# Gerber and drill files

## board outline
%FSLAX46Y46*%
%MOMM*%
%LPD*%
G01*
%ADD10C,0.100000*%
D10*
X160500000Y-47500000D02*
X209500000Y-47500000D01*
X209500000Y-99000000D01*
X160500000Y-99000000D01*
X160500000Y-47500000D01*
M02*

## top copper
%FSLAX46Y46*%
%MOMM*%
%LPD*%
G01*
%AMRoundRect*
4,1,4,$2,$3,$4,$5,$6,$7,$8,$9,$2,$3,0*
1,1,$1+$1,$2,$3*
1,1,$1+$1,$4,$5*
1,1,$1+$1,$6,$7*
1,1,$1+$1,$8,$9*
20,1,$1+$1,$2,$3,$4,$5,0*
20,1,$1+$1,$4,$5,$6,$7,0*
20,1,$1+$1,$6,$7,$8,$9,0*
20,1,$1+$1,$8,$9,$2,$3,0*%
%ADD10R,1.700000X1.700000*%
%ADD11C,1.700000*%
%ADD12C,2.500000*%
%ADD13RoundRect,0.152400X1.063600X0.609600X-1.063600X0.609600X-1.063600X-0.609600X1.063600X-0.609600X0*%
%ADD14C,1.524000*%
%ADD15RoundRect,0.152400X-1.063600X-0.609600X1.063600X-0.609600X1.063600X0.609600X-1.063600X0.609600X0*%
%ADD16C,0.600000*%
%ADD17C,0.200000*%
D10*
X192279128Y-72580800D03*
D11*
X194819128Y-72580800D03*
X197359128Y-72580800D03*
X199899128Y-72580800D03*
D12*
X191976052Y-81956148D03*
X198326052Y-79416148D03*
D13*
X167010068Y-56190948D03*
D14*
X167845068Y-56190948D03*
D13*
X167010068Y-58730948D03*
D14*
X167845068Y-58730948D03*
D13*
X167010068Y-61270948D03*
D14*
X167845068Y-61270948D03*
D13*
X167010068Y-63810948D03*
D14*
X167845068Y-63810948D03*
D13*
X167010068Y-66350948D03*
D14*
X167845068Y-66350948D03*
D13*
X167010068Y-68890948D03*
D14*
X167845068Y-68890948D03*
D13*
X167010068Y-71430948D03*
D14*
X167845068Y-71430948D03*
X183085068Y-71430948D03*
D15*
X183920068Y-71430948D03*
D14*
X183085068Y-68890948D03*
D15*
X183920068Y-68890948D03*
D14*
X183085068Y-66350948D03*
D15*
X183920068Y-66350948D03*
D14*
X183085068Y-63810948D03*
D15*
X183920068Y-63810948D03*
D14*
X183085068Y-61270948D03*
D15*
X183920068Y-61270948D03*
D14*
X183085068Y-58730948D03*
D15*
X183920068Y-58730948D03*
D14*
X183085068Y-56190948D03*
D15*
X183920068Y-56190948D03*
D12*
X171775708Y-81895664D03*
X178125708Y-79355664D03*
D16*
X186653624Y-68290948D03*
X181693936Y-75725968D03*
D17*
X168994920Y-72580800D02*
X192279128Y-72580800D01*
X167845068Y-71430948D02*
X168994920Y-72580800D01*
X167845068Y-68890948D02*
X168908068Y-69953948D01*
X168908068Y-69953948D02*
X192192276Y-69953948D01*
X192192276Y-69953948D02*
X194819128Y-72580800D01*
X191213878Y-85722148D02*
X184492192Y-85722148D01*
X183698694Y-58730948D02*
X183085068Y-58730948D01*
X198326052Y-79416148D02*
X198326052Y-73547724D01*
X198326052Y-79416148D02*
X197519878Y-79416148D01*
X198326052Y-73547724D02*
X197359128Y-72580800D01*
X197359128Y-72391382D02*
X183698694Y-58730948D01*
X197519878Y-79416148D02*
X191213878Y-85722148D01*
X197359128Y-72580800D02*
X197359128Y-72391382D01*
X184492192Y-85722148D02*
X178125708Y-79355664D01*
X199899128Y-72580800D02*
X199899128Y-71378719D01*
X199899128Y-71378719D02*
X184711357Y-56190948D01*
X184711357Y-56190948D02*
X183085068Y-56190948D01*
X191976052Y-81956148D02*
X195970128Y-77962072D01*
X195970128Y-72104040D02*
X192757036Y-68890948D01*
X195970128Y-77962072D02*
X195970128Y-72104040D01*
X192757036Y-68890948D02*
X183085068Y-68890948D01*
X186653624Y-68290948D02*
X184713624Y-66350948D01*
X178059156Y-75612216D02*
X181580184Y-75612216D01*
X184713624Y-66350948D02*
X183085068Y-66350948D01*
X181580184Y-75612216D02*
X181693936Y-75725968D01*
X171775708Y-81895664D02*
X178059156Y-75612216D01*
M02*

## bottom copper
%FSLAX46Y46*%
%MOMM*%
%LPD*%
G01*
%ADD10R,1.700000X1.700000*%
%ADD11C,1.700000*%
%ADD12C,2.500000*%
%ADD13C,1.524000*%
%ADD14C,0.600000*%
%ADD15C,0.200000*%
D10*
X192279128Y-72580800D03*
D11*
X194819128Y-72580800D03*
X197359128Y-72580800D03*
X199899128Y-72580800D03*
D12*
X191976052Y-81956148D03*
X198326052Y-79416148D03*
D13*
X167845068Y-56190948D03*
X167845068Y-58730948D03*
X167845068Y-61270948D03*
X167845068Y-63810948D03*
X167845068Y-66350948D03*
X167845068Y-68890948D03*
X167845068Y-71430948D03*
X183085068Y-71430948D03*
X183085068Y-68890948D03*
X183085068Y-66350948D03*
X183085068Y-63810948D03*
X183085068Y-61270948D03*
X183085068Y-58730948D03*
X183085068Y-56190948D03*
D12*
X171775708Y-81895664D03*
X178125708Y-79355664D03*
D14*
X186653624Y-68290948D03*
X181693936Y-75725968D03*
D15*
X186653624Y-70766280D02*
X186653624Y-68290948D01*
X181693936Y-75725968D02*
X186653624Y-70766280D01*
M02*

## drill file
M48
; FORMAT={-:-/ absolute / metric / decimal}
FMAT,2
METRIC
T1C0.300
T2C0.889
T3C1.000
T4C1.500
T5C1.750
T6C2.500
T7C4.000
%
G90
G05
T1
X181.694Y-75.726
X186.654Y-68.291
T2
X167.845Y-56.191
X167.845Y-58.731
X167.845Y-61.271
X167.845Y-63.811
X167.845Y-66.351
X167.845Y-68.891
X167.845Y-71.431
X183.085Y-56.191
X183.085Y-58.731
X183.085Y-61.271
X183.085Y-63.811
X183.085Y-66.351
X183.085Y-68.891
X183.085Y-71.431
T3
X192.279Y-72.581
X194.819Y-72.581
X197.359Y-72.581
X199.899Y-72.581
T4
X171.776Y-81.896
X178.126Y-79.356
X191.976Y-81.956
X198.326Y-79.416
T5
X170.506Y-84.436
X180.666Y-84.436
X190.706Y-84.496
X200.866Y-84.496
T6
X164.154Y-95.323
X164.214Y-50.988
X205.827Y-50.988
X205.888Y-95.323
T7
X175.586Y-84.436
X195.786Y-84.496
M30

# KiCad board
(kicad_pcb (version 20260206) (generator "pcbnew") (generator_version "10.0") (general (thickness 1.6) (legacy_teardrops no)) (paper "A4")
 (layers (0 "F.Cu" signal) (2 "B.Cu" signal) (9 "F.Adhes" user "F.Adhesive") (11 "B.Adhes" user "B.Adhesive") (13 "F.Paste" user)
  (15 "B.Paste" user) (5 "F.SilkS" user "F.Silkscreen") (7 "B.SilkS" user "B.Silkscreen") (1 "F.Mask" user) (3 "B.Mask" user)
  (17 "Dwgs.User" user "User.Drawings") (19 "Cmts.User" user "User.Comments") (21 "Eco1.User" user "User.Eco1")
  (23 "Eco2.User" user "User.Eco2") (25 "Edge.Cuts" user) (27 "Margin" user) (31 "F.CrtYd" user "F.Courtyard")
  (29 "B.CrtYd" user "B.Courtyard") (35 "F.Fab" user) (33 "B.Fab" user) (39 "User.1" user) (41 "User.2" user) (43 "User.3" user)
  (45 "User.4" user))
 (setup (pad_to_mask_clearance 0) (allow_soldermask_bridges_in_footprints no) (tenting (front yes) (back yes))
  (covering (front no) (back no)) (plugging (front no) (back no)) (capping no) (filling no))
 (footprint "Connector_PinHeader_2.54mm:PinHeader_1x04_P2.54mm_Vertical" (layer "F.Cu") (at 192.279128 72.5808 90)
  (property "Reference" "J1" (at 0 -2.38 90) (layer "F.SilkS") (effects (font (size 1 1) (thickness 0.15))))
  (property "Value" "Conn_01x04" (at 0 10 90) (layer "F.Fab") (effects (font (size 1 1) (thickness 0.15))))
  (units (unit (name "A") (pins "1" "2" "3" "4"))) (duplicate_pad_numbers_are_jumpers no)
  (pad "1" thru_hole rect (at 0 0 90) (size 1.7 1.7) (drill 1) (layers "*.Cu" "*.Mask") (remove_unused_layers no) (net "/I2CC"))
  (pad "2" thru_hole circle (at 0 2.54 90) (size 1.7 1.7) (drill 1) (layers "*.Cu" "*.Mask") (remove_unused_layers no) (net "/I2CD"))
  (pad "3" thru_hole circle (at 0 5.08 90) (size 1.7 1.7) (drill 1) (layers "*.Cu" "*.Mask") (remove_unused_layers no) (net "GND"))
  (pad "4" thru_hole circle (at 0 7.62 90) (size 1.7 1.7) (drill 1) (layers "*.Cu" "*.Mask") (remove_unused_layers no) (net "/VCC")))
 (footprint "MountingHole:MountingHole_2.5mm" (layer "F.Cu") (at 164.21406 50.988012)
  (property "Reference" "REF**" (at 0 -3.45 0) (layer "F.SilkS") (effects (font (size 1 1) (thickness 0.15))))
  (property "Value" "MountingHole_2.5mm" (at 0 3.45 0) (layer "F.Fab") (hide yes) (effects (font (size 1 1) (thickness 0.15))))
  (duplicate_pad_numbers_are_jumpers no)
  (pad "" np_thru_hole circle (at 0 0) (size 2.5 2.5) (drill 2.5) (layers "*.Cu" "*.Mask")))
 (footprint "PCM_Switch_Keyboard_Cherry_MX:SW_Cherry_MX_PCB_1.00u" (layer "F.Cu") (at 195.786052 84.496148)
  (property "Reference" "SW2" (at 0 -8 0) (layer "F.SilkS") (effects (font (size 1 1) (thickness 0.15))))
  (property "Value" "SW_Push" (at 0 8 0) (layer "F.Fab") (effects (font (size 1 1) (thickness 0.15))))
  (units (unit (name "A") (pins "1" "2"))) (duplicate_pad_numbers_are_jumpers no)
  (pad "" np_thru_hole circle (at -5.08 0) (size 1.75 1.75) (drill 1.75) (layers "*.Cu" "*.Mask"))
  (pad "" np_thru_hole circle (at 0 0) (size 4 4) (drill 4) (layers "*.Cu" "*.Mask"))
  (pad "" np_thru_hole circle (at 5.08 0) (size 1.75 1.75) (drill 1.75) (layers "*.Cu" "*.Mask"))
  (pad "1" thru_hole circle (at -3.81 -2.54) (size 2.5 2.5) (drill 1.5) (layers "*.Cu" "*.Mask") (remove_unused_layers no)
   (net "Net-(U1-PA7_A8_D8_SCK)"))
  (pad "2" thru_hole circle (at 2.54 -5.08) (size 2.5 2.5) (drill 1.5) (layers "*.Cu" "*.Mask") (remove_unused_layers no) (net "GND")))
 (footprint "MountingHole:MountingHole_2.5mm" (layer "F.Cu") (at 164.153576 95.322784)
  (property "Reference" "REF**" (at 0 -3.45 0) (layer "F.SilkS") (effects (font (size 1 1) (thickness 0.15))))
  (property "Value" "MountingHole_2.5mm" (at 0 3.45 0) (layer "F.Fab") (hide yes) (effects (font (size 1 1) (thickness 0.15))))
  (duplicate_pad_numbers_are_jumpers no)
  (pad "" np_thru_hole circle (at 0 0) (size 2.5 2.5) (drill 2.5) (layers "*.Cu" "*.Mask")))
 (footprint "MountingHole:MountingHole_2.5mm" (layer "F.Cu") (at 205.827052 50.988012)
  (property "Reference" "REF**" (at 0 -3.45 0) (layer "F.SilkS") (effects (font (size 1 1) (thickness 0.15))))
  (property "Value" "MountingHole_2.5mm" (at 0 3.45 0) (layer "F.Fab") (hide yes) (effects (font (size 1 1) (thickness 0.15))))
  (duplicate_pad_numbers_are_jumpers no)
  (pad "" np_thru_hole circle (at 0 0) (size 2.5 2.5) (drill 2.5) (layers "*.Cu" "*.Mask")))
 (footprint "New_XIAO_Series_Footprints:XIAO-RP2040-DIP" (layer "F.Cu") (at 175.465068 63.810948 90)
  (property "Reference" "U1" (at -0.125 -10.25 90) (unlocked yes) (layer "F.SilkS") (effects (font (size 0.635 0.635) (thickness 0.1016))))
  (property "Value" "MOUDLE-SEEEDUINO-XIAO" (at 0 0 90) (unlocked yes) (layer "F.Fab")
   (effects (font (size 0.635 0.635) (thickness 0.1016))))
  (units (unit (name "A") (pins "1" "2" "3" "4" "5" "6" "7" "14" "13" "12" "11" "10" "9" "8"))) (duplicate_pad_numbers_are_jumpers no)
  (pad "1" smd roundrect (at 7.62 -8.455 180) (size 2.432 1.524) (layers "F.Cu" "F.Mask") (roundrect_rratio 0.1)
   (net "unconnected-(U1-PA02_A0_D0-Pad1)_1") (thermal_bridge_angle 45))
  (pad "1" thru_hole circle (at 7.62 -7.62 180) (size 1.524 1.524) (drill 0.889) (layers "*.Cu" "*.Mask") (remove_unused_layers no)
   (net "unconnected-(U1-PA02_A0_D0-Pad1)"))
  (pad "2" smd roundrect (at 5.08 -8.455 180) (size 2.432 1.524) (layers "F.Cu" "F.Mask") (roundrect_rratio 0.1)
   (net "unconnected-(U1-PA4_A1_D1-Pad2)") (thermal_bridge_angle 45))
  (pad "2" thru_hole circle (at 5.08 -7.62 180) (size 1.524 1.524) (drill 0.889) (layers "*.Cu" "*.Mask") (remove_unused_layers no)
   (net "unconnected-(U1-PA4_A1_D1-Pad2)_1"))
  (pad "3" smd roundrect (at 2.54 -8.455 180) (size 2.432 1.524) (layers "F.Cu" "F.Mask") (roundrect_rratio 0.1)
   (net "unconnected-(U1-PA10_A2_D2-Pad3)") (thermal_bridge_angle 45))
  (pad "3" thru_hole circle (at 2.54 -7.62 180) (size 1.524 1.524) (drill 0.889) (layers "*.Cu" "*.Mask") (remove_unused_layers no)
   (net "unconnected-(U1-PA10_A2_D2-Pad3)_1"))
  (pad "4" smd roundrect (at 0 -8.455 180) (size 2.432 1.524) (layers "F.Cu" "F.Mask") (roundrect_rratio 0.1)
   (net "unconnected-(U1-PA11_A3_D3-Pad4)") (thermal_bridge_angle 45))
  (pad "4" thru_hole circle (at 0 -7.62 180) (size 1.524 1.524) (drill 0.889) (layers "*.Cu" "*.Mask") (remove_unused_layers no)
   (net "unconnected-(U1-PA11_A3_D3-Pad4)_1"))
  (pad "5" smd roundrect (at -2.54 -8.455 180) (size 2.432 1.524) (layers "F.Cu" "F.Mask") (roundrect_rratio 0.1)
   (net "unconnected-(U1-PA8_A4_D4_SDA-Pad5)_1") (thermal_bridge_angle 45))
  (pad "5" thru_hole circle (at -2.54 -7.62 180) (size 1.524 1.524) (drill 0.889) (layers "*.Cu" "*.Mask") (remove_unused_layers no)
   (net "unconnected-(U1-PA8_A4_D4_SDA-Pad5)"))
  (pad "6" smd roundrect (at -5.08 -8.455 180) (size 2.432 1.524) (layers "F.Cu" "F.Mask") (roundrect_rratio 0.1) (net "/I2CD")
   (thermal_bridge_angle 45))
  (pad "6" thru_hole circle (at -5.08 -7.62 180) (size 1.524 1.524) (drill 0.889) (layers "*.Cu" "*.Mask") (remove_unused_layers no)
   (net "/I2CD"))
  (pad "7" smd roundrect (at -7.62 -8.455 180) (size 2.432 1.524) (layers "F.Cu" "F.Mask") (roundrect_rratio 0.1) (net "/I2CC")
   (thermal_bridge_angle 45))
  (pad "7" thru_hole circle (at -7.62 -7.62 180) (size 1.524 1.524) (drill 0.889) (layers "*.Cu" "*.Mask") (remove_unused_layers no)
   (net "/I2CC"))
  (pad "8" thru_hole circle (at -7.62 7.62) (size 1.524 1.524) (drill 0.889) (layers "*.Cu" "*.Mask") (remove_unused_layers no)
   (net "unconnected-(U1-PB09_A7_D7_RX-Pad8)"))
  (pad "8" smd roundrect (at -7.62 8.455) (size 2.432 1.524) (layers "F.Cu" "F.Mask") (roundrect_rratio 0.1)
   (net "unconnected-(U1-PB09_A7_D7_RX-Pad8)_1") (thermal_bridge_angle 45))
  (pad "9" thru_hole circle (at -5.08 7.62) (size 1.524 1.524) (drill 0.889) (layers "*.Cu" "*.Mask") (remove_unused_layers no)
   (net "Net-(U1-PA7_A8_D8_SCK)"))
  (pad "9" smd roundrect (at -5.08 8.455) (size 2.432 1.524) (layers "F.Cu" "F.Mask") (roundrect_rratio 0.1) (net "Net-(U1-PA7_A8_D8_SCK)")
   (thermal_bridge_angle 45))
  (pad "10" thru_hole circle (at -2.54 7.62) (size 1.524 1.524) (drill 0.889) (layers "*.Cu" "*.Mask") (remove_unused_layers no)
   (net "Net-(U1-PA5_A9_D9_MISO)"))
  (pad "10" smd roundrect (at -2.54 8.455) (size 2.432 1.524) (layers "F.Cu" "F.Mask") (roundrect_rratio 0.1)
   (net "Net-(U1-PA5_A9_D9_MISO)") (thermal_bridge_angle 45))
  (pad "11" thru_hole circle (at 0 7.62) (size 1.524 1.524) (drill 0.889) (layers "*.Cu" "*.Mask") (remove_unused_layers no)
   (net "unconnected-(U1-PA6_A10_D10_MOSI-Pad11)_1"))
  (pad "11" smd roundrect (at 0 8.455) (size 2.432 1.524) (layers "F.Cu" "F.Mask") (roundrect_rratio 0.1)
   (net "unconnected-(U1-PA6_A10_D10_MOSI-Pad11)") (thermal_bridge_angle 45))
  (pad "12" thru_hole circle (at 2.54 7.62) (size 1.524 1.524) (drill 0.889) (layers "*.Cu" "*.Mask") (remove_unused_layers no)
   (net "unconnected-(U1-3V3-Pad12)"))
  (pad "12" smd roundrect (at 2.54 8.455) (size 2.432 1.524) (layers "F.Cu" "F.Mask") (roundrect_rratio 0.1)
   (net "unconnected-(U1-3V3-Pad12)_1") (thermal_bridge_angle 45))
  (pad "13" thru_hole circle (at 5.08 7.62) (size 1.524 1.524) (drill 0.889) (layers "*.Cu" "*.Mask") (remove_unused_layers no) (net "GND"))
  (pad "13" smd roundrect (at 5.08 8.455) (size 2.432 1.524) (layers "F.Cu" "F.Mask") (roundrect_rratio 0.1) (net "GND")
   (thermal_bridge_angle 45))
  (pad "14" thru_hole circle (at 7.62 7.62) (size 1.524 1.524) (drill 0.889) (layers "*.Cu" "*.Mask") (remove_unused_layers no) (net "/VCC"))
  (pad "14" smd roundrect (at 7.62 8.455) (size 2.432 1.524) (layers "F.Cu" "F.Mask") (roundrect_rratio 0.1) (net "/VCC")
   (thermal_bridge_angle 45)))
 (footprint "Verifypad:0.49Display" (layer "F.Cu") (at 193.609284 63.20578)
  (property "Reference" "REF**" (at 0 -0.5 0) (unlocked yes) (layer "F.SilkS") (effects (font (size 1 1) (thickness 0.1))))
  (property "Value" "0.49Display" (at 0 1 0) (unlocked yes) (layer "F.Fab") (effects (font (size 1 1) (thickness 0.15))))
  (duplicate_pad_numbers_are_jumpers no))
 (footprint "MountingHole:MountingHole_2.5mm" (layer "F.Cu") (at 205.887536 95.322784)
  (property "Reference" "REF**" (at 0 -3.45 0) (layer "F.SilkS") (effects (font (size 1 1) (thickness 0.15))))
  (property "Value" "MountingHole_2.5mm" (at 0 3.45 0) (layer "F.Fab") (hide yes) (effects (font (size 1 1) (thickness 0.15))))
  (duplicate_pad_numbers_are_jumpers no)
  (pad "" np_thru_hole circle (at 0 0) (size 2.5 2.5) (drill 2.5) (layers "*.Cu" "*.Mask")))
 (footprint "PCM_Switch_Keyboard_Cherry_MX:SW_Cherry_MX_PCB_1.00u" (layer "F.Cu") (at 175.585708 84.435664)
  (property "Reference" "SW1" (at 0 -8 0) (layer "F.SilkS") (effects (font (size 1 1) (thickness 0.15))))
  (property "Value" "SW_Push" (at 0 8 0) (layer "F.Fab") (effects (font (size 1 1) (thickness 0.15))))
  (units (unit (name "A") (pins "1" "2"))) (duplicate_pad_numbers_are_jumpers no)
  (pad "" np_thru_hole circle (at -5.08 0) (size 1.75 1.75) (drill 1.75) (layers "*.Cu" "*.Mask"))
  (pad "" np_thru_hole circle (at 0 0) (size 4 4) (drill 4) (layers "*.Cu" "*.Mask"))
  (pad "" np_thru_hole circle (at 5.08 0) (size 1.75 1.75) (drill 1.75) (layers "*.Cu" "*.Mask"))
  (pad "1" thru_hole circle (at -3.81 -2.54) (size 2.5 2.5) (drill 1.5) (layers "*.Cu" "*.Mask") (remove_unused_layers no)
   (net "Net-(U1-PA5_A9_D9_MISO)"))
  (pad "2" thru_hole circle (at 2.54 -5.08) (size 2.5 2.5) (drill 1.5) (layers "*.Cu" "*.Mask") (remove_unused_layers no) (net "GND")))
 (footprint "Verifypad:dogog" (layer "B.Cu") (at 175.734887 92.160269 180)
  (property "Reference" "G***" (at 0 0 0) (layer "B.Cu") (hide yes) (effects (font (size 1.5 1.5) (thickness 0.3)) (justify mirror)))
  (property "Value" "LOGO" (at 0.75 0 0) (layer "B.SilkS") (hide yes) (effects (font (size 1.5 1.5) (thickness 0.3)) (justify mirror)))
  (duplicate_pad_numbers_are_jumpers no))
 (gr_rect (start 160.5 47.5) (end 209.5 99) (stroke (width 0.1) (type solid)) (fill no) (layer "Edge.Cuts"))
 (segment (start 168.99492 72.5808) (end 192.279128 72.5808) (width 0.2) (layer "F.Cu") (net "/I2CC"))
 (segment (start 167.845068 71.430948) (end 168.99492 72.5808) (width 0.2) (layer "F.Cu") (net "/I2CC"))
 (segment (start 167.845068 68.890948) (end 168.908068 69.953948) (width 0.2) (layer "F.Cu") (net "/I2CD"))
 (segment (start 168.908068 69.953948) (end 192.192276 69.953948) (width 0.2) (layer "F.Cu") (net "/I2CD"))
 (segment (start 192.192276 69.953948) (end 194.819128 72.5808) (width 0.2) (layer "F.Cu") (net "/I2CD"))
 (segment (start 191.213878 85.722148) (end 184.492192 85.722148) (width 0.2) (layer "F.Cu") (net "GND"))
 (segment (start 183.698694 58.730948) (end 183.085068 58.730948) (width 0.2) (layer "F.Cu") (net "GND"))
 (segment (start 198.326052 79.416148) (end 198.326052 73.547724) (width 0.2) (layer "F.Cu") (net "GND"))
 (segment (start 198.326052 79.416148) (end 197.519878 79.416148) (width 0.2) (layer "F.Cu") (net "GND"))
 (segment (start 198.326052 73.547724) (end 197.359128 72.5808) (width 0.2) (layer "F.Cu") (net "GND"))
 (segment (start 197.359128 72.391382) (end 183.698694 58.730948) (width 0.2) (layer "F.Cu") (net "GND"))
 (segment (start 197.519878 79.416148) (end 191.213878 85.722148) (width 0.2) (layer "F.Cu") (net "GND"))
 (segment (start 197.359128 72.5808) (end 197.359128 72.391382) (width 0.2) (layer "F.Cu") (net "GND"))
 (segment (start 184.492192 85.722148) (end 178.125708 79.355664) (width 0.2) (layer "F.Cu") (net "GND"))
 (segment (start 199.899128 72.5808) (end 199.899128 71.378719) (width 0.2) (layer "F.Cu") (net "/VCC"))
 (segment (start 199.899128 71.378719) (end 184.711357 56.190948) (width 0.2) (layer "F.Cu") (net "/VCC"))
 (segment (start 184.711357 56.190948) (end 183.085068 56.190948) (width 0.2) (layer "F.Cu") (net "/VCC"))
 (segment (start 191.976052 81.956148) (end 195.970128 77.962072) (width 0.2) (layer "F.Cu") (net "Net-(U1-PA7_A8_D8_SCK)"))
 (segment (start 195.970128 72.10404) (end 192.757036 68.890948) (width 0.2) (layer "F.Cu") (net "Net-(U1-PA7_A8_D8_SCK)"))
 (segment (start 195.970128 77.962072) (end 195.970128 72.10404) (width 0.2) (layer "F.Cu") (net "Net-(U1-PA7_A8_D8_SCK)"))
 (segment (start 192.757036 68.890948) (end 183.085068 68.890948) (width 0.2) (layer "F.Cu") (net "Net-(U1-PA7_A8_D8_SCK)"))
 (segment (start 186.653624 68.290948) (end 184.713624 66.350948) (width 0.2) (layer "F.Cu") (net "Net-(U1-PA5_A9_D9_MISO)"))
 (segment (start 178.059156 75.612216) (end 181.580184 75.612216) (width 0.2) (layer "F.Cu") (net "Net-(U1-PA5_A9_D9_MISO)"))
 (segment (start 184.713624 66.350948) (end 183.085068 66.350948) (width 0.2) (layer "F.Cu") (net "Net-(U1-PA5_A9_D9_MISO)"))
 (segment (start 181.580184 75.612216) (end 181.693936 75.725968) (width 0.2) (layer "F.Cu") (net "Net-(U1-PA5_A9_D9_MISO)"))
 (segment (start 171.775708 81.895664) (end 178.059156 75.612216) (width 0.2) (layer "F.Cu") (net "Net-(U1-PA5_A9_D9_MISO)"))
 (via (at 186.653624 68.290948) (size 0.6) (drill 0.3) (layers "F.Cu" "B.Cu") (capping no) (covering (front no) (back no))
  (plugging (front no) (back no)) (filling no) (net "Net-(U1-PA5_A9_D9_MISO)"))
 (via (at 181.693936 75.725968) (size 0.6) (drill 0.3) (layers "F.Cu" "B.Cu") (capping no) (covering (front no) (back no))
  (plugging (front no) (back no)) (filling no) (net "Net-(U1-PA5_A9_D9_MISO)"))
 (segment (start 186.653624 70.76628) (end 186.653624 68.290948) (width 0.2) (layer "B.Cu") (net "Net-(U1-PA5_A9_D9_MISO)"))
 (segment (start 181.693936 75.725968) (end 186.653624 70.76628) (width 0.2) (layer "B.Cu") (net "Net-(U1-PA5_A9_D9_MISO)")))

